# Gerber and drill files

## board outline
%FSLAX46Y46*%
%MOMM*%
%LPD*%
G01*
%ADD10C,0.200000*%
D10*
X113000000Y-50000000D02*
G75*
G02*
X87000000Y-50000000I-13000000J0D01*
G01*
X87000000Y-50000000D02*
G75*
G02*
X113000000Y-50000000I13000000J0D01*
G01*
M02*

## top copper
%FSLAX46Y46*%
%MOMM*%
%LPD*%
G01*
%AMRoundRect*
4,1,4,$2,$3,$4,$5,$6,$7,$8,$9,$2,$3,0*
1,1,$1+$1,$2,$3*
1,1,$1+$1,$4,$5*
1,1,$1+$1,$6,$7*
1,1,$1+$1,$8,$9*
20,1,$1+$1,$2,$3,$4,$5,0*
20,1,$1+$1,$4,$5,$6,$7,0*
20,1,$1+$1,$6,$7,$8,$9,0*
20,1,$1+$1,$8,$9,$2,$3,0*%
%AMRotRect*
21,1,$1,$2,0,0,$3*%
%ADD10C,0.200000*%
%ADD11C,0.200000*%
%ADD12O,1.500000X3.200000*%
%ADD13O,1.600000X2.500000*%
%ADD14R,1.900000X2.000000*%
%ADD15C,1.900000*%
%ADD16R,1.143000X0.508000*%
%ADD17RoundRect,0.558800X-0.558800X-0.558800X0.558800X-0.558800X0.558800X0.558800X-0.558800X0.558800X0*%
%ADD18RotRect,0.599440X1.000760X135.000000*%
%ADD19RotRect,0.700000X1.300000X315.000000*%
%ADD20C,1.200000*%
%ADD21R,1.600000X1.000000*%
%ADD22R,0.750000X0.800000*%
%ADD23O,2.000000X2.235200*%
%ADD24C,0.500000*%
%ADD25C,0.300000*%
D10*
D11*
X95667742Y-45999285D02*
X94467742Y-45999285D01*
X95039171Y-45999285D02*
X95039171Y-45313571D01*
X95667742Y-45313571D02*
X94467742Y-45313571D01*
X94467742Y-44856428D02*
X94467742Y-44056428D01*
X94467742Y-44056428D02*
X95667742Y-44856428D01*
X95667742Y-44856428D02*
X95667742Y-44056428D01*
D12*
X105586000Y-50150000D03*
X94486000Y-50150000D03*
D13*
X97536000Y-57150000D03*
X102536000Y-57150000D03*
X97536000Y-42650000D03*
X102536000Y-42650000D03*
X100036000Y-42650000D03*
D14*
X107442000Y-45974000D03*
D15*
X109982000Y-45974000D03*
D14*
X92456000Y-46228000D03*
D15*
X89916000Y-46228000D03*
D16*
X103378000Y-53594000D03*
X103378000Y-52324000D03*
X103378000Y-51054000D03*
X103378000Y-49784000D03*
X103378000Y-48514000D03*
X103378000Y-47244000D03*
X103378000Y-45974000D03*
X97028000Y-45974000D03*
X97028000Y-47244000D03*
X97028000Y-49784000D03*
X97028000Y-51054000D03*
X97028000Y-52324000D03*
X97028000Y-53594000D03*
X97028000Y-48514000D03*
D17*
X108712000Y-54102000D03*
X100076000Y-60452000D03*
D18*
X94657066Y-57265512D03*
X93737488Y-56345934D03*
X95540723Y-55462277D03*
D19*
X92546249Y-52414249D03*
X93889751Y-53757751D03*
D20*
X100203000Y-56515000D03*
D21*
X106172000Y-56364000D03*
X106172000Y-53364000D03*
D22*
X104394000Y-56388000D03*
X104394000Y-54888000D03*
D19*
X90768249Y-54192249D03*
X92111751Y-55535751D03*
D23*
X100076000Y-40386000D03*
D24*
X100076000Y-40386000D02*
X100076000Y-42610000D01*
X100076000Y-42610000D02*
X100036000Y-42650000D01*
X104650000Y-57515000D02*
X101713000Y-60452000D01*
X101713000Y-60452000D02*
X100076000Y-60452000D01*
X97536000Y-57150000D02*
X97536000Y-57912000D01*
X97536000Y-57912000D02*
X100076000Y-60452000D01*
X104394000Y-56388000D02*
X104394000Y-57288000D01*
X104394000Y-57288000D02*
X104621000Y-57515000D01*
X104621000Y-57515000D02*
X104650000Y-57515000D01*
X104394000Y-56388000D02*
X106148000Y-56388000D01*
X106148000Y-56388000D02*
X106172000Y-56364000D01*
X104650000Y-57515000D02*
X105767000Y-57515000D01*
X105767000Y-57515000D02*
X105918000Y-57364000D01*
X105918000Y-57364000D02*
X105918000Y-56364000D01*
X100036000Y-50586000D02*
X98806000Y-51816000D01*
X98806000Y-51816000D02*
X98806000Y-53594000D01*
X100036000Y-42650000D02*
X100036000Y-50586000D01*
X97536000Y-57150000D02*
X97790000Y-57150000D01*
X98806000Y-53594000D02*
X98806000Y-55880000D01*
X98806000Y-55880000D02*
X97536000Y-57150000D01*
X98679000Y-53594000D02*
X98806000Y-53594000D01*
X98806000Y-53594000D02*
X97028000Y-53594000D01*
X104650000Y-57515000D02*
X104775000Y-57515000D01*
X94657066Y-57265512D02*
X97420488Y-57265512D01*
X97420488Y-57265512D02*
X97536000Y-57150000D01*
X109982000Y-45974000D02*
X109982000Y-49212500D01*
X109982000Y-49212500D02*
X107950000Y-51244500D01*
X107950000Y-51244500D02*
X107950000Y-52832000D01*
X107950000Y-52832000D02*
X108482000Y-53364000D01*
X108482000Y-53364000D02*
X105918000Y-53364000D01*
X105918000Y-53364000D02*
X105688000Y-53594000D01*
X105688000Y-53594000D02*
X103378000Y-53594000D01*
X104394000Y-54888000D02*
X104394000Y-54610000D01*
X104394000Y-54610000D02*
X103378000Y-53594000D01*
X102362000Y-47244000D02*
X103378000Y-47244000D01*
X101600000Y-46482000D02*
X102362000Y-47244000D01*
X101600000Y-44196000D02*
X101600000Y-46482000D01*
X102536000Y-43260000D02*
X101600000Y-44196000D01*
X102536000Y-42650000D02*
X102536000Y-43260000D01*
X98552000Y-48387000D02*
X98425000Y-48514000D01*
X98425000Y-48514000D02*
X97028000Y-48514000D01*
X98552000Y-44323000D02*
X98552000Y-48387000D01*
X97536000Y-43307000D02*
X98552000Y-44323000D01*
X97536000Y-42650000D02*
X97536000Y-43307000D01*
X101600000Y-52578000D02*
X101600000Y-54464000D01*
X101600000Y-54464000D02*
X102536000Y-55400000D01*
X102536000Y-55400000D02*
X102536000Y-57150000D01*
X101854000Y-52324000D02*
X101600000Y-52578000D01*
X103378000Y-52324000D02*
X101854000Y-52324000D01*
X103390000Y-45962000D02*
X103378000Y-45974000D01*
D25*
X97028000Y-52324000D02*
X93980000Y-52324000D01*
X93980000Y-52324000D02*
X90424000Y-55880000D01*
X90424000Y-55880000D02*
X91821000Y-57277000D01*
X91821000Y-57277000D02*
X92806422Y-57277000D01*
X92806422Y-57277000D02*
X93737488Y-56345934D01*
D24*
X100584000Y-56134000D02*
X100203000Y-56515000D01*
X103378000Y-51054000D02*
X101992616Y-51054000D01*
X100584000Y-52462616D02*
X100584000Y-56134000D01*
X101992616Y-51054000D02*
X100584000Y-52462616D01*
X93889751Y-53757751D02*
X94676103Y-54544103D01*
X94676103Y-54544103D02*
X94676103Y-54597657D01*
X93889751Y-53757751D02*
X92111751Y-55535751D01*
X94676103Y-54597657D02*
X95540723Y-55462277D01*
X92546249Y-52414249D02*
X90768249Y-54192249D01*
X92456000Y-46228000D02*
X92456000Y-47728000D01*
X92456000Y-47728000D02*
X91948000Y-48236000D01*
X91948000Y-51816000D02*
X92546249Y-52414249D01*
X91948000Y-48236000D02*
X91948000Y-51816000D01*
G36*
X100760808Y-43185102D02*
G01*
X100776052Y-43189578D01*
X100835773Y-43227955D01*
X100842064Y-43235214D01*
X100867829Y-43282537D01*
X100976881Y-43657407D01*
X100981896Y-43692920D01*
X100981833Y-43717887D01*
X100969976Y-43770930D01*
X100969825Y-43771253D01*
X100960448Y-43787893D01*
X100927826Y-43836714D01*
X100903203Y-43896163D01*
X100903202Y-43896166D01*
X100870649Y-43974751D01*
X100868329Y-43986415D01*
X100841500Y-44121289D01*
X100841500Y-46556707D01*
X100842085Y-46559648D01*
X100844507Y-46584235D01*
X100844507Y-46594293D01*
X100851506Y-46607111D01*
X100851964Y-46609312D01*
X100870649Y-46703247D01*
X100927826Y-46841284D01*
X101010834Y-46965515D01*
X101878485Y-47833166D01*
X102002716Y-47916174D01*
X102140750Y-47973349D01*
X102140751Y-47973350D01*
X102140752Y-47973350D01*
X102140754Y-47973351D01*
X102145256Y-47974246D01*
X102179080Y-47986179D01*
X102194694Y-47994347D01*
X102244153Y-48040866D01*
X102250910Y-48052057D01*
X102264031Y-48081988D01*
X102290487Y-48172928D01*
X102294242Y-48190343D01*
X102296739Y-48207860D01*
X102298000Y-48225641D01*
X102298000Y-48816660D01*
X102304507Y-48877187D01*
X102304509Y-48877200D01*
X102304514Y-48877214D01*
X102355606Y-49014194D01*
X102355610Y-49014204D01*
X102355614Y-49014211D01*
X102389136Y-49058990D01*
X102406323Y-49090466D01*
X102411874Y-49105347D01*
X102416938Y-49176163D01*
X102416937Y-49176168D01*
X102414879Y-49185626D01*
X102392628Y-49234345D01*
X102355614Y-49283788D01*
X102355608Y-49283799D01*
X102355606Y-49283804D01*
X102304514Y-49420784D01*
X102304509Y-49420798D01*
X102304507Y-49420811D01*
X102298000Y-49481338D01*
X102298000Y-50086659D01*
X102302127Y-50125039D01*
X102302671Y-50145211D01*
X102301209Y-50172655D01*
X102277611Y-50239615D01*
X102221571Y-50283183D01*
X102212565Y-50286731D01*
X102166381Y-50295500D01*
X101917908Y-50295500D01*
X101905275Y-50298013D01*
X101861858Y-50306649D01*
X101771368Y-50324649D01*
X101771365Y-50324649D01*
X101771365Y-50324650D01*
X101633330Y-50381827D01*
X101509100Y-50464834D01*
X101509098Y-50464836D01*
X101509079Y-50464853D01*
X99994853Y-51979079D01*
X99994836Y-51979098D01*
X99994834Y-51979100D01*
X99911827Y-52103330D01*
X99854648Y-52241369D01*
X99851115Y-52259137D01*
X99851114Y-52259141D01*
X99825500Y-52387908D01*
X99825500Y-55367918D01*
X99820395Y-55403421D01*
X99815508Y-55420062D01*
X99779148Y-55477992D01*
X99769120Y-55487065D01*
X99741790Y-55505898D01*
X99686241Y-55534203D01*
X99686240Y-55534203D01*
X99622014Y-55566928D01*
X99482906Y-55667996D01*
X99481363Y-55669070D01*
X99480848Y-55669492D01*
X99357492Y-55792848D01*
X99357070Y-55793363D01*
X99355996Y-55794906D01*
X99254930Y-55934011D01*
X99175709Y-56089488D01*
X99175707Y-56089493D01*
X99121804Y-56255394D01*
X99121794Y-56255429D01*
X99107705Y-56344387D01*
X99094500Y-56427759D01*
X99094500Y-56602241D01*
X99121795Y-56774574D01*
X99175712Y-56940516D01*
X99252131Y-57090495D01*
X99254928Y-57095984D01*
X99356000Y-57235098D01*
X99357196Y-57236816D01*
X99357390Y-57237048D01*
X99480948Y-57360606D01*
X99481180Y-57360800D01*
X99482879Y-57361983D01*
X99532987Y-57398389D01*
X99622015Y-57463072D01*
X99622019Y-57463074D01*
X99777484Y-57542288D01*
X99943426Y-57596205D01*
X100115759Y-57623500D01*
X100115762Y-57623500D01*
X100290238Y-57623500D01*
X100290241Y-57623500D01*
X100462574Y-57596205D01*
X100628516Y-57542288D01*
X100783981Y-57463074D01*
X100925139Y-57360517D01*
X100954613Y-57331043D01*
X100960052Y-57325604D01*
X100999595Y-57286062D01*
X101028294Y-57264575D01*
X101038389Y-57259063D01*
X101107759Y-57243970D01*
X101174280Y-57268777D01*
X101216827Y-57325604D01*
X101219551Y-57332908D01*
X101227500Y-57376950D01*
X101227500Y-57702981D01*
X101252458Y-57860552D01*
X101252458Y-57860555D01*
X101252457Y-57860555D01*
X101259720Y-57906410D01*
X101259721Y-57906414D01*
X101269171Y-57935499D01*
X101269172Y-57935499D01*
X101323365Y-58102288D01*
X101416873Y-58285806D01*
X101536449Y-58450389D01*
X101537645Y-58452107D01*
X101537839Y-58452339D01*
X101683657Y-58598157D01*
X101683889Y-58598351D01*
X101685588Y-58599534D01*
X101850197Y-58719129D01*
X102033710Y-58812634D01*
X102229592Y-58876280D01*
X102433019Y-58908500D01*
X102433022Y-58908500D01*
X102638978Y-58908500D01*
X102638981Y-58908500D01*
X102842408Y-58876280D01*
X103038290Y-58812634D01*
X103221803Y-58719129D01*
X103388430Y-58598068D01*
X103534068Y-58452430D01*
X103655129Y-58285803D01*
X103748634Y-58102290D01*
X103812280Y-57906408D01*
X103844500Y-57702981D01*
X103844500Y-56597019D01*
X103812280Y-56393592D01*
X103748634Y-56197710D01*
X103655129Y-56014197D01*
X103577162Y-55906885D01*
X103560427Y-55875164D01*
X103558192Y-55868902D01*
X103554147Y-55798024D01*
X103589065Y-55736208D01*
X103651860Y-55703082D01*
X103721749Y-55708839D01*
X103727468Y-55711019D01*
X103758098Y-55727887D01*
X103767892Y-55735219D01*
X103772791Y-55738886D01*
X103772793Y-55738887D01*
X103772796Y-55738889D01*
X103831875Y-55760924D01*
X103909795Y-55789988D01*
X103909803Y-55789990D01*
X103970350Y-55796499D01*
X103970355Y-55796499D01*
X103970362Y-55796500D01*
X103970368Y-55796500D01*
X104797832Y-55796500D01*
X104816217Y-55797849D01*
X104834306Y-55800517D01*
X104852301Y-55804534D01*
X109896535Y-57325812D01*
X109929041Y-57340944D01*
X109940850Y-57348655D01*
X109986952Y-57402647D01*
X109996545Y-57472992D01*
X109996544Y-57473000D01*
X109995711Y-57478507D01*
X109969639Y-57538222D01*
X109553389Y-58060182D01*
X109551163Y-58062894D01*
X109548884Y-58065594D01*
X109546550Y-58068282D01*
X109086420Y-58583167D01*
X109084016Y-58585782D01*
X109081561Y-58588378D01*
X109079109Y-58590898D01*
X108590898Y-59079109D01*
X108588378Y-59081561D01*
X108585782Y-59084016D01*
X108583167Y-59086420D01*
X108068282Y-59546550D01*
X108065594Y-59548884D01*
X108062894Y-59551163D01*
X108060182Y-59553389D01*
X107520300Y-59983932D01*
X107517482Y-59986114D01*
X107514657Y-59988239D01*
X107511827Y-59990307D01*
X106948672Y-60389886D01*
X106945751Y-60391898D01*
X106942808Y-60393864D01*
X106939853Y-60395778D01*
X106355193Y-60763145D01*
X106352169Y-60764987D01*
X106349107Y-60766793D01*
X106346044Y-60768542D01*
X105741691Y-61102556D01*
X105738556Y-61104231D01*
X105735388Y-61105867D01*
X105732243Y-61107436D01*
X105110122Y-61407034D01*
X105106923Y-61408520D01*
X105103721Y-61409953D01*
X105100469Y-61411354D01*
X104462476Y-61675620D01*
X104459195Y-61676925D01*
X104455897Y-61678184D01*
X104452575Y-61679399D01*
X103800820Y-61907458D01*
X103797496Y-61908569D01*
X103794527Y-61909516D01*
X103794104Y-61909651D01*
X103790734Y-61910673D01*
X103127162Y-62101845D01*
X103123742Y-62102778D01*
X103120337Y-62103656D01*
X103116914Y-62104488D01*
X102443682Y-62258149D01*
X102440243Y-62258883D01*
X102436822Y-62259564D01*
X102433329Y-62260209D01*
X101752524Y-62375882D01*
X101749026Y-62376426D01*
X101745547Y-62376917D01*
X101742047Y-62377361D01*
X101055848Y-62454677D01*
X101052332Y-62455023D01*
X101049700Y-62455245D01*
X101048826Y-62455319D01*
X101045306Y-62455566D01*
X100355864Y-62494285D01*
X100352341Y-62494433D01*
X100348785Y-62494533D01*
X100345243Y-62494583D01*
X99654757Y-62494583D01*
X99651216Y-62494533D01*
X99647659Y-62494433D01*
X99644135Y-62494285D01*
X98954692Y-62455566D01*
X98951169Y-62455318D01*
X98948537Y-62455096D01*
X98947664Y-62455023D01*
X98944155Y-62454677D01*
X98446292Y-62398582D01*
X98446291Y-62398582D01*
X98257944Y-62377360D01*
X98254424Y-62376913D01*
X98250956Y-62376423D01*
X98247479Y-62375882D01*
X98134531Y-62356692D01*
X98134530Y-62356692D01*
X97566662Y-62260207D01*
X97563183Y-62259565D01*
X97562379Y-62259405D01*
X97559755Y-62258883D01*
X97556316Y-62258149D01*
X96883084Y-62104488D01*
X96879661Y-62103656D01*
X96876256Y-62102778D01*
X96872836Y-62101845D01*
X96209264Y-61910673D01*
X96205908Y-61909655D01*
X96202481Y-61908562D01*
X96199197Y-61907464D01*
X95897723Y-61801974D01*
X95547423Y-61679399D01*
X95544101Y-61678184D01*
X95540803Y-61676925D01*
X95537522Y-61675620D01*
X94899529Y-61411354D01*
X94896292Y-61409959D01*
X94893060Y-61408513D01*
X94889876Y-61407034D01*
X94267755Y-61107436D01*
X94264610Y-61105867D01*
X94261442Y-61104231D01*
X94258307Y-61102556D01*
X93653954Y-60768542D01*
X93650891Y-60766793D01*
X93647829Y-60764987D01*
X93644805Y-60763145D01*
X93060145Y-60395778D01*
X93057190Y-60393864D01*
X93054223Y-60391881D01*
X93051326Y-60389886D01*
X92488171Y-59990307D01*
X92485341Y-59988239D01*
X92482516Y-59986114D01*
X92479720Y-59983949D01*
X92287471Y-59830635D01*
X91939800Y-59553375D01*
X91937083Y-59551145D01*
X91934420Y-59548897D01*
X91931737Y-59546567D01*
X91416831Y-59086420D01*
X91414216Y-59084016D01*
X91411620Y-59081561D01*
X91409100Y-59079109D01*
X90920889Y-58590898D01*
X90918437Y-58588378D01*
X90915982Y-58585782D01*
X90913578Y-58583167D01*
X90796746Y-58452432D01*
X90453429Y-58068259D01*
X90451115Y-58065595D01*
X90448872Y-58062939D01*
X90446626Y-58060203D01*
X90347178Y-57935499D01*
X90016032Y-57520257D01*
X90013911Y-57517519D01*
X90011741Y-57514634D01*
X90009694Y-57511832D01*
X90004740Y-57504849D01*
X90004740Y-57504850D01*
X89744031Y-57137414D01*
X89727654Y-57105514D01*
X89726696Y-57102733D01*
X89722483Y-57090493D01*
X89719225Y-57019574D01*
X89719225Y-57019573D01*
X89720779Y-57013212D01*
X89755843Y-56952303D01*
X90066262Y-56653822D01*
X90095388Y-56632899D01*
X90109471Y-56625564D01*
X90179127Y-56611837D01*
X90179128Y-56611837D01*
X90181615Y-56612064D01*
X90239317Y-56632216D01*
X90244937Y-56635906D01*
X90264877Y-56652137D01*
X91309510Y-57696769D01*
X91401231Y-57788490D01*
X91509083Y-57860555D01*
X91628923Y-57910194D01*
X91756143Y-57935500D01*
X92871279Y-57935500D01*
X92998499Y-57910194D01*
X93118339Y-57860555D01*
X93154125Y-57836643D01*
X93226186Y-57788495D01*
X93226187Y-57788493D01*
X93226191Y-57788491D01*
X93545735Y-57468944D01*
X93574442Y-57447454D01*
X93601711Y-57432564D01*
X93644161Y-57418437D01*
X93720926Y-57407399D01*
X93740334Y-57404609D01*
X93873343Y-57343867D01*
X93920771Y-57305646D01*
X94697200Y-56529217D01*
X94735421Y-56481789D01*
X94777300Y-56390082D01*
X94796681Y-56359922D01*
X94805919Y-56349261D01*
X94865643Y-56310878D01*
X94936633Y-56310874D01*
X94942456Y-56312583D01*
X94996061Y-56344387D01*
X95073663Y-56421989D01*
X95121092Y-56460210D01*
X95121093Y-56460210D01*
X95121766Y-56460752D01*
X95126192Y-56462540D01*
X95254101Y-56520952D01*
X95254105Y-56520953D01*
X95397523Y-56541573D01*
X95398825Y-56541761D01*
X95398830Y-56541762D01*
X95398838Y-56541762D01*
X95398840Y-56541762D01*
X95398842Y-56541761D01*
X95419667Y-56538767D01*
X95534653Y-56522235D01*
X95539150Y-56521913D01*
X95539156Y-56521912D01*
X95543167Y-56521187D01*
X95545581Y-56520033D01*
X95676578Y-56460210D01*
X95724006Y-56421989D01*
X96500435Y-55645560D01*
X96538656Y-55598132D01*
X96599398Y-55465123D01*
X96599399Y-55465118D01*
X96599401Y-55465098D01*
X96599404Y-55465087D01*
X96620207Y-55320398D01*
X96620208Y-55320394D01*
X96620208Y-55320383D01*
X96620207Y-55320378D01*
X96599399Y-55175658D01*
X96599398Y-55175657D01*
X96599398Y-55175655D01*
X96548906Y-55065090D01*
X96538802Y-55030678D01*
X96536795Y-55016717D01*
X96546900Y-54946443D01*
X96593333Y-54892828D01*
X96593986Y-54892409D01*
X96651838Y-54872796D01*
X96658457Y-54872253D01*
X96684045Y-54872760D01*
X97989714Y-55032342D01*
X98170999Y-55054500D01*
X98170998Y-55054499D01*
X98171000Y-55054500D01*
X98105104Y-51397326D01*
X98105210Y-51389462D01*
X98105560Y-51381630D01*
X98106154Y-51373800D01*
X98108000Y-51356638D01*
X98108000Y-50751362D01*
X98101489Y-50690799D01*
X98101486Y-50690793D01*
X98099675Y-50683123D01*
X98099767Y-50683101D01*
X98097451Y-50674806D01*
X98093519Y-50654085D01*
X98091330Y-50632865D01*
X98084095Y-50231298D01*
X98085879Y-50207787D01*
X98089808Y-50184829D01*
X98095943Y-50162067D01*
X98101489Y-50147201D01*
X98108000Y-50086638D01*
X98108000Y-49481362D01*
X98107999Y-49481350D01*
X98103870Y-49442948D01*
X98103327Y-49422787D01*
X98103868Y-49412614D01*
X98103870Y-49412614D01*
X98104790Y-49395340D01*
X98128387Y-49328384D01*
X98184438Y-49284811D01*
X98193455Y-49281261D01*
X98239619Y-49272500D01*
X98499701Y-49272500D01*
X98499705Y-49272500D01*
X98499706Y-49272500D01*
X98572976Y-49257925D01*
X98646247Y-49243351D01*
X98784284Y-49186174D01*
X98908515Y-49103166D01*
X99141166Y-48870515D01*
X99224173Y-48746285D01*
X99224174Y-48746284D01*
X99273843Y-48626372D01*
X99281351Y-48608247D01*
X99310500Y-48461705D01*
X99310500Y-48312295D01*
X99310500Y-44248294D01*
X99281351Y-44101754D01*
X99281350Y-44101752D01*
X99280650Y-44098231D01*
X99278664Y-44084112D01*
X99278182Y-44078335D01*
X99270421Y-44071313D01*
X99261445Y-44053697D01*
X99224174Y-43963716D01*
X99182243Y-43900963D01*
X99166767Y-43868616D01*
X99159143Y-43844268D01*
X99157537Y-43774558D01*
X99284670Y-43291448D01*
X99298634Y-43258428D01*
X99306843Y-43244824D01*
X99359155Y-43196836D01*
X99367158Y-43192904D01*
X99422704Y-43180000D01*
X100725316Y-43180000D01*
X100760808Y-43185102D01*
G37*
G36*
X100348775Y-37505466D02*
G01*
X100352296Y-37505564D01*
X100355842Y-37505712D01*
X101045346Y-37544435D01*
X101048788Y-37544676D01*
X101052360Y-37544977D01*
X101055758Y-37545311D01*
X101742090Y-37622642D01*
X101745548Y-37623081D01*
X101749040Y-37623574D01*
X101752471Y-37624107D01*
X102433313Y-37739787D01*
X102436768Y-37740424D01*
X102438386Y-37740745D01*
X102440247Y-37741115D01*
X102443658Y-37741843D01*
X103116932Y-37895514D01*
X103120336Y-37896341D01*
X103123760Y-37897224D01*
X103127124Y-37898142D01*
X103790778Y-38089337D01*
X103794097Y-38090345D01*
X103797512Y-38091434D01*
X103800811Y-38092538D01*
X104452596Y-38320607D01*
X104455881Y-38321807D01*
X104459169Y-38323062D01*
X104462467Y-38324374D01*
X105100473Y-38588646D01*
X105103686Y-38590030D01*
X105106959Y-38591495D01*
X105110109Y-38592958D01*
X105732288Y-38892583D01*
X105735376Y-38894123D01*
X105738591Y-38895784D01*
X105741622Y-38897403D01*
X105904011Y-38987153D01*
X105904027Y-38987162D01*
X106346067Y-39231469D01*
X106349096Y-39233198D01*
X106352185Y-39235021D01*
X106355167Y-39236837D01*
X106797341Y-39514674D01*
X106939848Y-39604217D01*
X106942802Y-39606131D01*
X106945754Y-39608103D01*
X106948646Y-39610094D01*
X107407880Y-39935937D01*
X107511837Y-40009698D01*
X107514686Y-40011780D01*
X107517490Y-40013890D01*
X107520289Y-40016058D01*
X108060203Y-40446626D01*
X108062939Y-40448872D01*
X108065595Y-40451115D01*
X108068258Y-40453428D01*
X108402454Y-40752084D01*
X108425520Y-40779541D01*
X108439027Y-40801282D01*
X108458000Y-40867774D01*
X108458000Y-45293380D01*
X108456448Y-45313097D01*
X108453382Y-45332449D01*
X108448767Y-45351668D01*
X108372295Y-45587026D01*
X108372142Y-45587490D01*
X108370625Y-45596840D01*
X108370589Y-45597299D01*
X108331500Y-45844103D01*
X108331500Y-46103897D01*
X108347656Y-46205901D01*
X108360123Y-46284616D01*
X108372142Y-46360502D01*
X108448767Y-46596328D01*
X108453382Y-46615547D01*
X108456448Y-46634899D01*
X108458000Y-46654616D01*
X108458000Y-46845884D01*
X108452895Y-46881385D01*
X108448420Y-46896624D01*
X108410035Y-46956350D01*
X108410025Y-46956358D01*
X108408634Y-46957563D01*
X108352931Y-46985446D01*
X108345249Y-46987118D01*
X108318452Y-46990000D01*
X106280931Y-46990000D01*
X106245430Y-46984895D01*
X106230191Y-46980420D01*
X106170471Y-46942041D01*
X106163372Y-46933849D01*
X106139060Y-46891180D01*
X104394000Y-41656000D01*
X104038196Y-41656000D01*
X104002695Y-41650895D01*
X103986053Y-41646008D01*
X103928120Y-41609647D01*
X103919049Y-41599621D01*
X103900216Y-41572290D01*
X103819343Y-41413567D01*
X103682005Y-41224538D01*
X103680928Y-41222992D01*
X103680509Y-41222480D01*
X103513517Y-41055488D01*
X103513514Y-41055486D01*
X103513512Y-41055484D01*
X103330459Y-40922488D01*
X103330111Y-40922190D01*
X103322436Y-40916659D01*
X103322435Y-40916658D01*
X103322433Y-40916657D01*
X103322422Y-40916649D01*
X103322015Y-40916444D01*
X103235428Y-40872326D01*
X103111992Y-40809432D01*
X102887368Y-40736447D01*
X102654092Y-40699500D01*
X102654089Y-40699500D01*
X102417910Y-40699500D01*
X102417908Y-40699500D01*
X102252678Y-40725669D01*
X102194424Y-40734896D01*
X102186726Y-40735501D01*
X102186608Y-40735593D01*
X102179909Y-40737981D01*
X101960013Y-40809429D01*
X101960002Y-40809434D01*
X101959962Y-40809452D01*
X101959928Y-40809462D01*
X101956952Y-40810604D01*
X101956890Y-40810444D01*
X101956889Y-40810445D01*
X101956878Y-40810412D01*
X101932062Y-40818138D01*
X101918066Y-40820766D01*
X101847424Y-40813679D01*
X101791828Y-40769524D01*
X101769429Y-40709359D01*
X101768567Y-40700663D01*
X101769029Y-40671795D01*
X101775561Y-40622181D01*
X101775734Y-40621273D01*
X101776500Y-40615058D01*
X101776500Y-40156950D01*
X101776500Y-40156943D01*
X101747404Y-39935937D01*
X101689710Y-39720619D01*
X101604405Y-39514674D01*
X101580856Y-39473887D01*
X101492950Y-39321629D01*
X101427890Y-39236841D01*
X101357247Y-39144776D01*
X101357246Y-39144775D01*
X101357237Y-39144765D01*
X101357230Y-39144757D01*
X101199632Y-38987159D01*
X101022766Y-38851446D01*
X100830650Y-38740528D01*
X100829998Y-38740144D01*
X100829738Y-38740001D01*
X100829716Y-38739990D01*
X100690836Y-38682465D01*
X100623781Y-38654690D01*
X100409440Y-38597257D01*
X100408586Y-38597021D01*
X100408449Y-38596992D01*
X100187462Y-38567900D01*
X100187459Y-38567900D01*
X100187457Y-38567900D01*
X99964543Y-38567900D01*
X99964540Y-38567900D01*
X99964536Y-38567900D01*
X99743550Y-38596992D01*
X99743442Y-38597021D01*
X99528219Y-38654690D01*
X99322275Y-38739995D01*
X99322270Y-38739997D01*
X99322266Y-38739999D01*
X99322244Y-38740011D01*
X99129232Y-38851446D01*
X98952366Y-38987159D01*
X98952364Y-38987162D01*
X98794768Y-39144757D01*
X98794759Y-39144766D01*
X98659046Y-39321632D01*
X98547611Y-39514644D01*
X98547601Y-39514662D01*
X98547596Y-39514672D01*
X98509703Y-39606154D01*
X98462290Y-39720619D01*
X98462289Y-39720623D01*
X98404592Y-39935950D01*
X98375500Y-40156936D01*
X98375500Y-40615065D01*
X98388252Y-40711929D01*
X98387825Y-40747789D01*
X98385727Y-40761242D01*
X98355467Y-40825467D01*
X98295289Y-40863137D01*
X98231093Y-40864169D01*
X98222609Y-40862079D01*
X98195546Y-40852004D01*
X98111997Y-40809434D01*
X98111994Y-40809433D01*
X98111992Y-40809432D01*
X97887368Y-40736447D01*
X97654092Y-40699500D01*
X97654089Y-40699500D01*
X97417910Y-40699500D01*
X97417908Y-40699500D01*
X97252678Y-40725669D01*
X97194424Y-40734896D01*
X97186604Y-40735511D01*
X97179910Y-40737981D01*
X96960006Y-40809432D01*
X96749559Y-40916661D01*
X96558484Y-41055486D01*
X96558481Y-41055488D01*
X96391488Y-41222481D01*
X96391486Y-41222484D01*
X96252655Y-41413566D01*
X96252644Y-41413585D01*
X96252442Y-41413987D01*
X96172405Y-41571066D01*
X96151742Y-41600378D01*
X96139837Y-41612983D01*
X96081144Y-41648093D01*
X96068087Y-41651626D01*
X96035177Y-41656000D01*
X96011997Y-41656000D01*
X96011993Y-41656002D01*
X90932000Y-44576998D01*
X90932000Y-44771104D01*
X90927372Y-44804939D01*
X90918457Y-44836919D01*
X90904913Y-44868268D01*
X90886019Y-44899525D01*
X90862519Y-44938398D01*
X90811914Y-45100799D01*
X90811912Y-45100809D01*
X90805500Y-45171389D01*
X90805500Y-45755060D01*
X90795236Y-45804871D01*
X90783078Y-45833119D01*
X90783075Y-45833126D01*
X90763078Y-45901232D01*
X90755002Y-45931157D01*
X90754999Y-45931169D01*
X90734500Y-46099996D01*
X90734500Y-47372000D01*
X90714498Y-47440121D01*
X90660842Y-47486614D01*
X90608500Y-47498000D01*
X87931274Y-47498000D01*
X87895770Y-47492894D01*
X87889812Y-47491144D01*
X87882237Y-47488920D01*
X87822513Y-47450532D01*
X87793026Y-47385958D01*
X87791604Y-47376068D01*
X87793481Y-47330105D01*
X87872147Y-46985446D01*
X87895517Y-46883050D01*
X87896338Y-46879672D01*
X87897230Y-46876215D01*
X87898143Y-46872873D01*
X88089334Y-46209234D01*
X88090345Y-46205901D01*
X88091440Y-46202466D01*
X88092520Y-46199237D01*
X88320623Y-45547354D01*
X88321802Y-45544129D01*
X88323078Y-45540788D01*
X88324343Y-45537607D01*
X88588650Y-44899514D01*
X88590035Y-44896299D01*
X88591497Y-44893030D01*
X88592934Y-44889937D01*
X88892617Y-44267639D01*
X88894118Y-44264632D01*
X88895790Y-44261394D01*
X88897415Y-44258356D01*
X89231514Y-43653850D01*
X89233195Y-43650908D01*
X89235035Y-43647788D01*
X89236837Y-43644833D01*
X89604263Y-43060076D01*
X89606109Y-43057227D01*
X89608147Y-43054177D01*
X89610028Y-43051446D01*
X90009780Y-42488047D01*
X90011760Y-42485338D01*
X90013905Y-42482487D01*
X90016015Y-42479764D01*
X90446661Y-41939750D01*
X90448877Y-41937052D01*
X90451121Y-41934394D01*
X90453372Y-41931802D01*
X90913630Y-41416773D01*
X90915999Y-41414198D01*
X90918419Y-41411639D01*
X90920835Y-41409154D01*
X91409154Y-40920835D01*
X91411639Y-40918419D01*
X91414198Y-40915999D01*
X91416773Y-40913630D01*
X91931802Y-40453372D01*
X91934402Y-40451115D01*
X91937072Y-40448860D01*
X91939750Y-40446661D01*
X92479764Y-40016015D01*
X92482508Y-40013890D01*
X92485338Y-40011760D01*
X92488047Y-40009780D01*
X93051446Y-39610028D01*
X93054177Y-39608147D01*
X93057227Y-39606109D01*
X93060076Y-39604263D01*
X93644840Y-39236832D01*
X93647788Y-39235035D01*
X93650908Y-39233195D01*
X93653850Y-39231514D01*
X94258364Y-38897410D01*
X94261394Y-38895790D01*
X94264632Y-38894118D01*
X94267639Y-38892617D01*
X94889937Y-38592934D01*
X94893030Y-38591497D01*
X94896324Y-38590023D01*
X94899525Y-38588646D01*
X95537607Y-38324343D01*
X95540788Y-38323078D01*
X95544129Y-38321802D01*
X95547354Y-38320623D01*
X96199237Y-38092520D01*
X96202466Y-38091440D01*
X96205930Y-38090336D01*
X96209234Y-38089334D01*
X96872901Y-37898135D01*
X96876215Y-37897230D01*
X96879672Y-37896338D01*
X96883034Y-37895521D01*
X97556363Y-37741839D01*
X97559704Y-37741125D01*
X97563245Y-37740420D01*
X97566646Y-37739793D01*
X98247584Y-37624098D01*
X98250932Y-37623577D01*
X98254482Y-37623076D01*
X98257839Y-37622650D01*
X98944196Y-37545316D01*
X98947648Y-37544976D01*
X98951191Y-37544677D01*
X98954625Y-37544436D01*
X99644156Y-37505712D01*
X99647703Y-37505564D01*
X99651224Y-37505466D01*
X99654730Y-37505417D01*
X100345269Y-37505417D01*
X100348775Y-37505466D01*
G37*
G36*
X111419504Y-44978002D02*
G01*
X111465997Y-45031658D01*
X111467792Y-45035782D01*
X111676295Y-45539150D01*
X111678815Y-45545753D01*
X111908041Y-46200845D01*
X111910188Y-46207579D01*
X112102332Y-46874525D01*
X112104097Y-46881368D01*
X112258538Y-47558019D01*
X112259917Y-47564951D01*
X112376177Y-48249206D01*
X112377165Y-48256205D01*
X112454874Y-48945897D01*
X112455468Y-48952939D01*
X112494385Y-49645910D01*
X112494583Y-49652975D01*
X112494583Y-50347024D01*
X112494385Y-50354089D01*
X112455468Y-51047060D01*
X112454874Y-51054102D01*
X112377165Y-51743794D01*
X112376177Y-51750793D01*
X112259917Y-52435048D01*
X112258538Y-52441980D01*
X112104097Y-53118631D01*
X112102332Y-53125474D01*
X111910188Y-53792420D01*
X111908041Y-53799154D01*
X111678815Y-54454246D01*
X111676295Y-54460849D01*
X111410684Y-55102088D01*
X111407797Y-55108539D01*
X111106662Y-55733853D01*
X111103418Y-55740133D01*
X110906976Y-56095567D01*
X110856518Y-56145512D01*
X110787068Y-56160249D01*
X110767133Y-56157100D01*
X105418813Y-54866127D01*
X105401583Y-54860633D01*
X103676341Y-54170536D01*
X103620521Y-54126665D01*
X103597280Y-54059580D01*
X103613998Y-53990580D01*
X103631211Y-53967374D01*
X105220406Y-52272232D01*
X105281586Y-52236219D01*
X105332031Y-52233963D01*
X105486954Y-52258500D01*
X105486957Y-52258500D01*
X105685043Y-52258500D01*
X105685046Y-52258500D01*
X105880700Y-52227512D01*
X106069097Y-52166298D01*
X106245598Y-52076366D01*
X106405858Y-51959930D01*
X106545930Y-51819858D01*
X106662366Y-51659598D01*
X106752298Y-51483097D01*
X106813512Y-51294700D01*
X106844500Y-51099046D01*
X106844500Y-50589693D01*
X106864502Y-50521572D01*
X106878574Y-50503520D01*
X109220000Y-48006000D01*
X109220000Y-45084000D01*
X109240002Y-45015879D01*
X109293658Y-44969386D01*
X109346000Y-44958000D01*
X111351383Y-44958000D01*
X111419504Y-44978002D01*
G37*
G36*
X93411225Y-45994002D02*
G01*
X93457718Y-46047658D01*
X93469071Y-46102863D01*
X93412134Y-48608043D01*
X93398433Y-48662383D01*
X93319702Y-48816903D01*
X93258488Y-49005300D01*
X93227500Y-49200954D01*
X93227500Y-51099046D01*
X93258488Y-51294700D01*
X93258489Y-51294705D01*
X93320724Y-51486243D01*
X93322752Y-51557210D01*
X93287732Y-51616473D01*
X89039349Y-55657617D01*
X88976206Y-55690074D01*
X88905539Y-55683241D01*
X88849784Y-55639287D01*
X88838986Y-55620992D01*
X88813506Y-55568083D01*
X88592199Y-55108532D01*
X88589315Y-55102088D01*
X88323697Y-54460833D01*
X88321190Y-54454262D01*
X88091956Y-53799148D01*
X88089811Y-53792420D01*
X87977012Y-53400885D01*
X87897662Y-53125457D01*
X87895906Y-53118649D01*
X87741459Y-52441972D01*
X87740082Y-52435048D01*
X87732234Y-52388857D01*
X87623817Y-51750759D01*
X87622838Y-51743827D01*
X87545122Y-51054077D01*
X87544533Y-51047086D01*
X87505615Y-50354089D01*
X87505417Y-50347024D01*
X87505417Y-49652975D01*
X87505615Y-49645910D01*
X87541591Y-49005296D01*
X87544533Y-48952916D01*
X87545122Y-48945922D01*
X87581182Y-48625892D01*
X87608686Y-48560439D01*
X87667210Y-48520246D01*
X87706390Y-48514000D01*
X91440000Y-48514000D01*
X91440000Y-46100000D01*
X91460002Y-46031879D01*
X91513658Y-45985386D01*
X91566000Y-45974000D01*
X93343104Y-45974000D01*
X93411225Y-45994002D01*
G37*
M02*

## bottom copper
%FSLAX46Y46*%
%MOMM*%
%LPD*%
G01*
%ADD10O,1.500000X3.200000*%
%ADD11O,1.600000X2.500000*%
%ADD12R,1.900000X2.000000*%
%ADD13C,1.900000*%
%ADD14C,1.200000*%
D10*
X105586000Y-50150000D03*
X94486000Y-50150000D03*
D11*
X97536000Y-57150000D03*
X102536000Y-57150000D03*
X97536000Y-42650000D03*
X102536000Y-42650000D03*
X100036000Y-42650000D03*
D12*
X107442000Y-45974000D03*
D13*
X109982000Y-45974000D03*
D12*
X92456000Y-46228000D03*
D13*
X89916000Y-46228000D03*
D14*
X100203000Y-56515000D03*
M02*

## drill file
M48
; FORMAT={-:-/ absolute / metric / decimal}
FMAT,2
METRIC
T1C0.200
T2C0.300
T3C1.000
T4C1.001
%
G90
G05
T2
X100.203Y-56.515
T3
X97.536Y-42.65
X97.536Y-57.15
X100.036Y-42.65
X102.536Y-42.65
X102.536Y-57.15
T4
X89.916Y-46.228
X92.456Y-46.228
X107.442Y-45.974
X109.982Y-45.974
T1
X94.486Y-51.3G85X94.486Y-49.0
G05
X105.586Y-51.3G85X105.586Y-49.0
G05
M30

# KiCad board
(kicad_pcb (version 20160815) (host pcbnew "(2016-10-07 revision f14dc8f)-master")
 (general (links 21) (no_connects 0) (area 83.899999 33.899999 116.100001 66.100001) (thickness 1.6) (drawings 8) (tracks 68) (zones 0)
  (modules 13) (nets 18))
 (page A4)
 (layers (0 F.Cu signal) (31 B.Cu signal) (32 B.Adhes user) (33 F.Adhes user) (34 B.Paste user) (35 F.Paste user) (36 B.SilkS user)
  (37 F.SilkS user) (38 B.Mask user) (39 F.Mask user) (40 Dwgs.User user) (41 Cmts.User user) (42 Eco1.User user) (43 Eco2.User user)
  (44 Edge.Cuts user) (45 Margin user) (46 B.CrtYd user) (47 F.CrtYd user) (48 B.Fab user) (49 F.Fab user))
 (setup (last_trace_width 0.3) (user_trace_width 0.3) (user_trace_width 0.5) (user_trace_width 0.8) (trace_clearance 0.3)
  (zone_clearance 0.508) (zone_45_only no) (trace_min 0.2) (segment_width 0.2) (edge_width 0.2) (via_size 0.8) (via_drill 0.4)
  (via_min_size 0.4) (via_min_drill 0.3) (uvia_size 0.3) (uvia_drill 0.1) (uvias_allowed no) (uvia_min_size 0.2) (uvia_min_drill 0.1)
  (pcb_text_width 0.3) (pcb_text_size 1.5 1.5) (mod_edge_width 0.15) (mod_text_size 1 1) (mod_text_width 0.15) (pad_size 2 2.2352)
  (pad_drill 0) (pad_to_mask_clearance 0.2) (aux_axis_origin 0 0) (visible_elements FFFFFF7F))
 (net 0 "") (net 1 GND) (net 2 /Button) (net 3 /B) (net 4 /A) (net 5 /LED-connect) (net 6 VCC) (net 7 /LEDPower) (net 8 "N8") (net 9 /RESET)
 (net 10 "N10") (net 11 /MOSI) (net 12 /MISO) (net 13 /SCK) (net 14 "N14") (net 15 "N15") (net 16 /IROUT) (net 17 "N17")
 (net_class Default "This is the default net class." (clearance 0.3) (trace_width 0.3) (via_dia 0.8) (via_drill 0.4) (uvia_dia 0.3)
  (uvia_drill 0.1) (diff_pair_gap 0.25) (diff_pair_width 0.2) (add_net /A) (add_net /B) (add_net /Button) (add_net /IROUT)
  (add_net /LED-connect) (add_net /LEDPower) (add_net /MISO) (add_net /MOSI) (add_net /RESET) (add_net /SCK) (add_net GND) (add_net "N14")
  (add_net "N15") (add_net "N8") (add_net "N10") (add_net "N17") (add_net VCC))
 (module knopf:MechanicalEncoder (layer B.Cu) (at 100.036 50.15 180)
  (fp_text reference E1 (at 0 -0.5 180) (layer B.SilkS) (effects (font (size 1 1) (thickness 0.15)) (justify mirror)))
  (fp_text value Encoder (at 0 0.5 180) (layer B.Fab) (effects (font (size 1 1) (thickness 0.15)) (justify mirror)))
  (pad 6 thru_hole oval (at -5.55 0 180) (size 1.5 3.2) (drill oval 0.2 2.5) (layers *.Cu *.Mask))
  (pad 6 thru_hole oval (at 5.55 0 180) (size 1.5 3.2) (drill oval 0.2 2.5) (layers *.Cu *.Mask))
  (pad 5 thru_hole oval (at 2.5 -7 180) (size 1.6 2.5) (drill 1) (layers *.Cu *.Mask) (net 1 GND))
  (pad 4 thru_hole oval (at -2.5 -7 180) (size 1.6 2.5) (drill 1) (layers *.Cu *.Mask) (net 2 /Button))
  (pad 3 thru_hole oval (at 2.5 7.5 180) (size 1.6 2.5) (drill 1) (layers *.Cu *.Mask) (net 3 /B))
  (pad 1 thru_hole oval (at -2.5 7.5 180) (size 1.6 2.5) (drill 1) (layers *.Cu *.Mask) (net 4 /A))
  (pad 2 thru_hole oval (at 0 7.5 180) (size 1.6 2.5) (drill 1) (layers *.Cu *.Mask) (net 1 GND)))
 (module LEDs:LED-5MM (layer F.Cu) (at 107.442 45.974)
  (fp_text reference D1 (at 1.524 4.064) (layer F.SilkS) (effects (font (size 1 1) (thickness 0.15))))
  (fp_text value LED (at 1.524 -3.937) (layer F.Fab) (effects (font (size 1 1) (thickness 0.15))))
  (pad 1 thru_hole rect (at 0 0 90) (size 2 1.9) (drill 1.00076) (layers *.Cu *.Mask F.SilkS) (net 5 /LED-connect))
  (pad 2 thru_hole circle (at 2.54 0) (size 1.9 1.9) (drill 1.00076) (layers *.Cu *.Mask F.SilkS) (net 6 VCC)))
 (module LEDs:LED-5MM (layer F.Cu) (at 92.456 46.228 180)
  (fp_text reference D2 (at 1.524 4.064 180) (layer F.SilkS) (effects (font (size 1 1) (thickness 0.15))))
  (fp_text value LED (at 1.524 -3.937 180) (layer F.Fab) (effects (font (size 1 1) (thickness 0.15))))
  (pad 1 thru_hole rect (at 0 0 270) (size 2 1.9) (drill 1.00076) (layers *.Cu *.Mask F.SilkS) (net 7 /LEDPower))
  (pad 2 thru_hole circle (at 2.54 0 180) (size 1.9 1.9) (drill 1.00076) (layers *.Cu *.Mask F.SilkS) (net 5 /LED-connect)))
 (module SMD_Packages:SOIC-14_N (layer F.Cu) (at 100.076 49.784 90)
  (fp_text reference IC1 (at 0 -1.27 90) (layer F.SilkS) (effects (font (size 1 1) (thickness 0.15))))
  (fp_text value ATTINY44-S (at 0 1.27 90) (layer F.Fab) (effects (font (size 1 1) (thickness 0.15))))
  (pad 1 smd rect (at -3.81 3.302 90) (size 0.508 1.143) (layers F.Cu F.Paste F.Mask) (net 6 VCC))
  (pad 2 smd rect (at -2.54 3.302 90) (size 0.508 1.143) (layers F.Cu F.Paste F.Mask) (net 2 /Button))
  (pad 3 smd rect (at -1.27 3.302 90) (size 0.508 1.143) (layers F.Cu F.Paste F.Mask) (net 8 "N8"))
  (pad 4 smd rect (at 0 3.302 90) (size 0.508 1.143) (layers F.Cu F.Paste F.Mask) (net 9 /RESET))
  (pad 5 smd rect (at 1.27 3.302 90) (size 0.508 1.143) (layers F.Cu F.Paste F.Mask) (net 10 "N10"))
  (pad 6 smd rect (at 2.54 3.302 90) (size 0.508 1.143) (layers F.Cu F.Paste F.Mask) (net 4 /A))
  (pad 7 smd rect (at 3.81 3.302 90) (size 0.508 1.143) (layers F.Cu F.Paste F.Mask) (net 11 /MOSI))
  (pad 8 smd rect (at 3.81 -3.048 90) (size 0.508 1.143) (layers F.Cu F.Paste F.Mask) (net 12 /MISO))
  (pad 9 smd rect (at 2.54 -3.048 90) (size 0.508 1.143) (layers F.Cu F.Paste F.Mask) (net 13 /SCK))
  (pad 11 smd rect (at 0 -3.048 90) (size 0.508 1.143) (layers F.Cu F.Paste F.Mask) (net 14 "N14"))
  (pad 12 smd rect (at -1.27 -3.048 90) (size 0.508 1.143) (layers F.Cu F.Paste F.Mask) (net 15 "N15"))
  (pad 13 smd rect (at -2.54 -3.048 90) (size 0.508 1.143) (layers F.Cu F.Paste F.Mask) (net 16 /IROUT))
  (pad 14 smd rect (at -3.81 -3.048 90) (size 0.508 1.143) (layers F.Cu F.Paste F.Mask) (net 1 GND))
  (pad 10 smd rect (at 1.27 -3.048 90) (size 0.508 1.143) (layers F.Cu F.Paste F.Mask) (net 3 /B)))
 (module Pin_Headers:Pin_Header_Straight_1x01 (layer F.Cu) (at 108.712 54.102)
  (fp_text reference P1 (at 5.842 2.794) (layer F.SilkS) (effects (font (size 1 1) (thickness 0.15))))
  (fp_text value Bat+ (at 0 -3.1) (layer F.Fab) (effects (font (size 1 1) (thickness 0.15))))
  (pad 1 smd roundrect (at 0 0) (size 2.2352 2.2352) (layers F.Cu F.Paste F.Mask) (roundrect_rratio 0.25) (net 6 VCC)))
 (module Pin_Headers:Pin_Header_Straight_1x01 (layer F.Cu) (at 100.076 60.452)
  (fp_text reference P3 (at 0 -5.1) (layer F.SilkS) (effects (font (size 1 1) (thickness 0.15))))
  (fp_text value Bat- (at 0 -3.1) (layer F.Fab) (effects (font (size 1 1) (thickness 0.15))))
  (pad 1 smd roundrect (at 0 0) (size 2.2352 2.2352) (layers F.Cu F.Paste F.Mask) (roundrect_rratio 0.25) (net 1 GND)))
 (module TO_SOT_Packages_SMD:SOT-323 (layer F.Cu) (at 94.869 56.134 135)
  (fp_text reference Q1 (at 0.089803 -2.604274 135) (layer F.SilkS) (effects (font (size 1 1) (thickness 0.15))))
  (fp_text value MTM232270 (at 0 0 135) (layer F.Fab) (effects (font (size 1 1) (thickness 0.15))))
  (pad 2 smd rect (at -0.65024 -0.94996 135) (size 0.59944 1.00076) (layers F.Cu F.Paste F.Mask) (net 1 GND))
  (pad 1 smd rect (at 0.65024 -0.94996 135) (size 0.59944 1.00076) (layers F.Cu F.Paste F.Mask) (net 16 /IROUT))
  (pad 3 smd rect (at 0 0.94996 135) (size 0.59944 1.00076) (layers F.Cu F.Paste F.Mask) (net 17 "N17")))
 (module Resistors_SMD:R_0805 (layer F.Cu) (at 93.218 53.086 315)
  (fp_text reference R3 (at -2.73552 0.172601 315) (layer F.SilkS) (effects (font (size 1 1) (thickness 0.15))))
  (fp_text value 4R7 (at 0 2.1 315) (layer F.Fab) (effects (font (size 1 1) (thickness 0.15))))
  (pad 1 smd rect (at -0.949999 0 315) (size 0.7 1.3) (layers F.Cu F.Paste F.Mask) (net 7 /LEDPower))
  (pad 2 smd rect (at 0.949999 0 315) (size 0.7 1.3) (layers F.Cu F.Paste F.Mask) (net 17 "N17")))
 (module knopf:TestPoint (layer F.Cu) (at 100.203 56.515)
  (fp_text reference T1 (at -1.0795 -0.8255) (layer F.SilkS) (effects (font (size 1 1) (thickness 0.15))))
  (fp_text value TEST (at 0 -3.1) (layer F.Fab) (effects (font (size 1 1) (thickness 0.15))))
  (pad 1 thru_hole circle (at 0 0) (size 1.2 1.2) (drill 0.3) (layers *.Cu *.Mask F.SilkS) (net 8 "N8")))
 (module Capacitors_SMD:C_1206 (layer F.Cu) (at 106.172 54.864 270)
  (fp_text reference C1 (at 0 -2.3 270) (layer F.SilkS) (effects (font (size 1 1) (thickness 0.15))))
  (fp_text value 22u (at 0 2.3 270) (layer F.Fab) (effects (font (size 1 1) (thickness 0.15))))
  (pad 2 smd rect (at 1.5 0 270) (size 1 1.6) (layers F.Cu F.Paste F.Mask) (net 1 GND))
  (pad 1 smd rect (at -1.5 0 270) (size 1 1.6) (layers F.Cu F.Paste F.Mask) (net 6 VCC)))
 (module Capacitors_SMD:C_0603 (layer F.Cu) (at 104.394 55.638 270)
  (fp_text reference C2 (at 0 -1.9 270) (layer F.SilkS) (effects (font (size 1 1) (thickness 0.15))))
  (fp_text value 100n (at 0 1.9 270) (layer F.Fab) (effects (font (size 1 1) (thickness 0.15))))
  (pad 2 smd rect (at 0.75 0 270) (size 0.8 0.75) (layers F.Cu F.Paste F.Mask) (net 1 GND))
  (pad 1 smd rect (at -0.75 0 270) (size 0.8 0.75) (layers F.Cu F.Paste F.Mask) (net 6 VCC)))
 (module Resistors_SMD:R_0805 (layer F.Cu) (at 91.44 54.864 315)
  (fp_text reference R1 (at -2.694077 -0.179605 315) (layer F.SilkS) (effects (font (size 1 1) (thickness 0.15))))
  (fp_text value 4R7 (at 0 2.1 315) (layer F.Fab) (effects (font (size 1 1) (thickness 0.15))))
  (pad 1 smd rect (at -0.949999 0 315) (size 0.7 1.3) (layers F.Cu F.Paste F.Mask) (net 7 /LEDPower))
  (pad 2 smd rect (at 0.949999 0 315) (size 0.7 1.3) (layers F.Cu F.Paste F.Mask) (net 17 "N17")))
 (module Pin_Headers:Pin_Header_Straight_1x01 (layer F.Cu) (at 100.076 40.386)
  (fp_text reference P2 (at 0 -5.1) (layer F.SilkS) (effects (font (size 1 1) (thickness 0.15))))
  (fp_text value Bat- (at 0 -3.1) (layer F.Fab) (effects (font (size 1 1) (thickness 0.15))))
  (pad 1 smd oval (at 0 0) (size 2 2.2352) (layers F.Cu F.Paste F.Mask) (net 1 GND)))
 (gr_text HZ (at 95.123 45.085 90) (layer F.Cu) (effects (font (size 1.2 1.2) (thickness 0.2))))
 (gr_circle (center 100 50) (end 113 50) (layer Edge.Cuts) (width 0.2))
 (segment (start 100.076 40.386) (end 100.076 42.61) (width 0.5) (layer F.Cu) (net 1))
 (segment (start 100.076 42.61) (end 100.036 42.65) (width 0.5) (layer F.Cu) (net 1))
 (segment (start 104.65 57.515) (end 101.713 60.452) (width 0.5) (layer F.Cu) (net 1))
 (segment (start 101.713 60.452) (end 100.076 60.452) (width 0.5) (layer F.Cu) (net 1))
 (segment (start 97.536 57.15) (end 97.536 57.912) (width 0.5) (layer F.Cu) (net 1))
 (segment (start 97.536 57.912) (end 100.076 60.452) (width 0.5) (layer F.Cu) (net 1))
 (segment (start 104.394 56.388) (end 104.394 57.288) (width 0.5) (layer F.Cu) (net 1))
 (segment (start 104.394 57.288) (end 104.621 57.515) (width 0.5) (layer F.Cu) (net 1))
 (segment (start 104.621 57.515) (end 104.65 57.515) (width 0.5) (layer F.Cu) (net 1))
 (segment (start 104.394 56.388) (end 106.148 56.388) (width 0.5) (layer F.Cu) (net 1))
 (segment (start 106.148 56.388) (end 106.172 56.364) (width 0.5) (layer F.Cu) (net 1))
 (segment (start 104.65 57.515) (end 105.767 57.515) (width 0.5) (layer F.Cu) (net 1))
 (segment (start 105.767 57.515) (end 105.918 57.364) (width 0.5) (layer F.Cu) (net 1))
 (segment (start 105.918 57.364) (end 105.918 56.364) (width 0.5) (layer F.Cu) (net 1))
 (segment (start 100.036 50.586) (end 98.806 51.816) (width 0.5) (layer F.Cu) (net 1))
 (segment (start 98.806 51.816) (end 98.806 53.594) (width 0.5) (layer F.Cu) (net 1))
 (segment (start 100.036 42.65) (end 100.036 50.586) (width 0.5) (layer F.Cu) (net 1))
 (segment (start 97.536 57.15) (end 97.79 57.15) (width 0.5) (layer F.Cu) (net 1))
 (segment (start 98.806 53.594) (end 98.806 55.88) (width 0.5) (layer F.Cu) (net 1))
 (segment (start 98.806 55.88) (end 97.536 57.15) (width 0.5) (layer F.Cu) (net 1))
 (segment (start 98.679 53.594) (end 98.806 53.594) (width 0.5) (layer F.Cu) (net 1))
 (segment (start 98.806 53.594) (end 97.028 53.594) (width 0.5) (layer F.Cu) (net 1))
 (segment (start 104.65 57.515) (end 104.775 57.515) (width 0.5) (layer F.Cu) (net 1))
 (segment (start 94.657066 57.265512) (end 97.420488 57.265512) (width 0.5) (layer F.Cu) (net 1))
 (segment (start 97.420488 57.265512) (end 97.536 57.15) (width 0.5) (layer F.Cu) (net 1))
 (segment (start 109.982 45.974) (end 109.982 49.2125) (width 0.5) (layer F.Cu) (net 6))
 (segment (start 109.982 49.2125) (end 107.95 51.2445) (width 0.5) (layer F.Cu) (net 6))
 (segment (start 107.95 51.2445) (end 107.95 52.832) (width 0.5) (layer F.Cu) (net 6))
 (segment (start 107.95 52.832) (end 108.482 53.364) (width 0.5) (layer F.Cu) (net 6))
 (segment (start 108.482 53.364) (end 105.918 53.364) (width 0.5) (layer F.Cu) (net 6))
 (segment (start 105.918 53.364) (end 105.688 53.594) (width 0.5) (layer F.Cu) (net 6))
 (segment (start 105.688 53.594) (end 103.378 53.594) (width 0.5) (layer F.Cu) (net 6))
 (segment (start 104.394 54.888) (end 104.394 54.61) (width 0.5) (layer F.Cu) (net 6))
 (segment (start 104.394 54.61) (end 103.378 53.594) (width 0.5) (layer F.Cu) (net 6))
 (segment (start 102.362 47.244) (end 103.378 47.244) (width 0.5) (layer F.Cu) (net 4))
 (segment (start 101.6 46.482) (end 102.362 47.244) (width 0.5) (layer F.Cu) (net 4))
 (segment (start 101.6 44.196) (end 101.6 46.482) (width 0.5) (layer F.Cu) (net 4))
 (segment (start 102.536 43.26) (end 101.6 44.196) (width 0.5) (layer F.Cu) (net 4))
 (segment (start 102.536 42.65) (end 102.536 43.26) (width 0.5) (layer F.Cu) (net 4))
 (segment (start 98.552 48.387) (end 98.425 48.514) (width 0.5) (layer F.Cu) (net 3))
 (segment (start 98.425 48.514) (end 97.028 48.514) (width 0.5) (layer F.Cu) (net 3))
 (segment (start 98.552 44.323) (end 98.552 48.387) (width 0.5) (layer F.Cu) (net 3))
 (segment (start 97.536 43.307) (end 98.552 44.323) (width 0.5) (layer F.Cu) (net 3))
 (segment (start 97.536 42.65) (end 97.536 43.307) (width 0.5) (layer F.Cu) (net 3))
 (segment (start 101.6 52.578) (end 101.6 54.464) (width 0.5) (layer F.Cu) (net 2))
 (segment (start 101.6 54.464) (end 102.536 55.4) (width 0.5) (layer F.Cu) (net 2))
 (segment (start 102.536 55.4) (end 102.536 57.15) (width 0.5) (layer F.Cu) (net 2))
 (segment (start 101.854 52.324) (end 101.6 52.578) (width 0.5) (layer F.Cu) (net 2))
 (segment (start 103.378 52.324) (end 101.854 52.324) (width 0.5) (layer F.Cu) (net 2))
 (segment (start 103.39 45.962) (end 103.378 45.974) (width 0.5) (layer F.Cu) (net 11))
 (segment (start 97.028 52.324) (end 93.98 52.324) (width 0.3) (layer F.Cu) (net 16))
 (segment (start 93.98 52.324) (end 90.424 55.88) (width 0.3) (layer F.Cu) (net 16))
 (segment (start 90.424 55.88) (end 91.821 57.277) (width 0.3) (layer F.Cu) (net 16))
 (segment (start 91.821 57.277) (end 92.806422 57.277) (width 0.3) (layer F.Cu) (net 16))
 (segment (start 92.806422 57.277) (end 93.737488 56.345934) (width 0.3) (layer F.Cu) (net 16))
 (segment (start 100.584 56.134) (end 100.203 56.515) (width 0.5) (layer F.Cu) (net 8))
 (segment (start 103.378 51.054) (end 101.992616 51.054) (width 0.5) (layer F.Cu) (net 8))
 (segment (start 100.584 52.462616) (end 100.584 56.134) (width 0.5) (layer F.Cu) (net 8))
 (segment (start 101.992616 51.054) (end 100.584 52.462616) (width 0.5) (layer F.Cu) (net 8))
 (segment (start 93.889751 53.757751) (end 94.676103 54.544103) (width 0.5) (layer F.Cu) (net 17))
 (segment (start 94.676103 54.544103) (end 94.676103 54.597657) (width 0.5) (layer F.Cu) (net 17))
 (segment (start 93.889751 53.757751) (end 92.111751 55.535751) (width 0.5) (layer F.Cu) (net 17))
 (segment (start 94.676103 54.597657) (end 95.540723 55.462277) (width 0.5) (layer F.Cu) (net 17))
 (segment (start 92.546249 52.414249) (end 90.768249 54.192249) (width 0.5) (layer F.Cu) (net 7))
 (segment (start 92.456 46.228) (end 92.456 47.728) (width 0.5) (layer F.Cu) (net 7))
 (segment (start 92.456 47.728) (end 91.948 48.236) (width 0.5) (layer F.Cu) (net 7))
 (segment (start 91.948 51.816) (end 92.546249 52.414249) (width 0.5) (layer F.Cu) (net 7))
 (segment (start 91.948 48.236) (end 91.948 51.816) (width 0.5) (layer F.Cu) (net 7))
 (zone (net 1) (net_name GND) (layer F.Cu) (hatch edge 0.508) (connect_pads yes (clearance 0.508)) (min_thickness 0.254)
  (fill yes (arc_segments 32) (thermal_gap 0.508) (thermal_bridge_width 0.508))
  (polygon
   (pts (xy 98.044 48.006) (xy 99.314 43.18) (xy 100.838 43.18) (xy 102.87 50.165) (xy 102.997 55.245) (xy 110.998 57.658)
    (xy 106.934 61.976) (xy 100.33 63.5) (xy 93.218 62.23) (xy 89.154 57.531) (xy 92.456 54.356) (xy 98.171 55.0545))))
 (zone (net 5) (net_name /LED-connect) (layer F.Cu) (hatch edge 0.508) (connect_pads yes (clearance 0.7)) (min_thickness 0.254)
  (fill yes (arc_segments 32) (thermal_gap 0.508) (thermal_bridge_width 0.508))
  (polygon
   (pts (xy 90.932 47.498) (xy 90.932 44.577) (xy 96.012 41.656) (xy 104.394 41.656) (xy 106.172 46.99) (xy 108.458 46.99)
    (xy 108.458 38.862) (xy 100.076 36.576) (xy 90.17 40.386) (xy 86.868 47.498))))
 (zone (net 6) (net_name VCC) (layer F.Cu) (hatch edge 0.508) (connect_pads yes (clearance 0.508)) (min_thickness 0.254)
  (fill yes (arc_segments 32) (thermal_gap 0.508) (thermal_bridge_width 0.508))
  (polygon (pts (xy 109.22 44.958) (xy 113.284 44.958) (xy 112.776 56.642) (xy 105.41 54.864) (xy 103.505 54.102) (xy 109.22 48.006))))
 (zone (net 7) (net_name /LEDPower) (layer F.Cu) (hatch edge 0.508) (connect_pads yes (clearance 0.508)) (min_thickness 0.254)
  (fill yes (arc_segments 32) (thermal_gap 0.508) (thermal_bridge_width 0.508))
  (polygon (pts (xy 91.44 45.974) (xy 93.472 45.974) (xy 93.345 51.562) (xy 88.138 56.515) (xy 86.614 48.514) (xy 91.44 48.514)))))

